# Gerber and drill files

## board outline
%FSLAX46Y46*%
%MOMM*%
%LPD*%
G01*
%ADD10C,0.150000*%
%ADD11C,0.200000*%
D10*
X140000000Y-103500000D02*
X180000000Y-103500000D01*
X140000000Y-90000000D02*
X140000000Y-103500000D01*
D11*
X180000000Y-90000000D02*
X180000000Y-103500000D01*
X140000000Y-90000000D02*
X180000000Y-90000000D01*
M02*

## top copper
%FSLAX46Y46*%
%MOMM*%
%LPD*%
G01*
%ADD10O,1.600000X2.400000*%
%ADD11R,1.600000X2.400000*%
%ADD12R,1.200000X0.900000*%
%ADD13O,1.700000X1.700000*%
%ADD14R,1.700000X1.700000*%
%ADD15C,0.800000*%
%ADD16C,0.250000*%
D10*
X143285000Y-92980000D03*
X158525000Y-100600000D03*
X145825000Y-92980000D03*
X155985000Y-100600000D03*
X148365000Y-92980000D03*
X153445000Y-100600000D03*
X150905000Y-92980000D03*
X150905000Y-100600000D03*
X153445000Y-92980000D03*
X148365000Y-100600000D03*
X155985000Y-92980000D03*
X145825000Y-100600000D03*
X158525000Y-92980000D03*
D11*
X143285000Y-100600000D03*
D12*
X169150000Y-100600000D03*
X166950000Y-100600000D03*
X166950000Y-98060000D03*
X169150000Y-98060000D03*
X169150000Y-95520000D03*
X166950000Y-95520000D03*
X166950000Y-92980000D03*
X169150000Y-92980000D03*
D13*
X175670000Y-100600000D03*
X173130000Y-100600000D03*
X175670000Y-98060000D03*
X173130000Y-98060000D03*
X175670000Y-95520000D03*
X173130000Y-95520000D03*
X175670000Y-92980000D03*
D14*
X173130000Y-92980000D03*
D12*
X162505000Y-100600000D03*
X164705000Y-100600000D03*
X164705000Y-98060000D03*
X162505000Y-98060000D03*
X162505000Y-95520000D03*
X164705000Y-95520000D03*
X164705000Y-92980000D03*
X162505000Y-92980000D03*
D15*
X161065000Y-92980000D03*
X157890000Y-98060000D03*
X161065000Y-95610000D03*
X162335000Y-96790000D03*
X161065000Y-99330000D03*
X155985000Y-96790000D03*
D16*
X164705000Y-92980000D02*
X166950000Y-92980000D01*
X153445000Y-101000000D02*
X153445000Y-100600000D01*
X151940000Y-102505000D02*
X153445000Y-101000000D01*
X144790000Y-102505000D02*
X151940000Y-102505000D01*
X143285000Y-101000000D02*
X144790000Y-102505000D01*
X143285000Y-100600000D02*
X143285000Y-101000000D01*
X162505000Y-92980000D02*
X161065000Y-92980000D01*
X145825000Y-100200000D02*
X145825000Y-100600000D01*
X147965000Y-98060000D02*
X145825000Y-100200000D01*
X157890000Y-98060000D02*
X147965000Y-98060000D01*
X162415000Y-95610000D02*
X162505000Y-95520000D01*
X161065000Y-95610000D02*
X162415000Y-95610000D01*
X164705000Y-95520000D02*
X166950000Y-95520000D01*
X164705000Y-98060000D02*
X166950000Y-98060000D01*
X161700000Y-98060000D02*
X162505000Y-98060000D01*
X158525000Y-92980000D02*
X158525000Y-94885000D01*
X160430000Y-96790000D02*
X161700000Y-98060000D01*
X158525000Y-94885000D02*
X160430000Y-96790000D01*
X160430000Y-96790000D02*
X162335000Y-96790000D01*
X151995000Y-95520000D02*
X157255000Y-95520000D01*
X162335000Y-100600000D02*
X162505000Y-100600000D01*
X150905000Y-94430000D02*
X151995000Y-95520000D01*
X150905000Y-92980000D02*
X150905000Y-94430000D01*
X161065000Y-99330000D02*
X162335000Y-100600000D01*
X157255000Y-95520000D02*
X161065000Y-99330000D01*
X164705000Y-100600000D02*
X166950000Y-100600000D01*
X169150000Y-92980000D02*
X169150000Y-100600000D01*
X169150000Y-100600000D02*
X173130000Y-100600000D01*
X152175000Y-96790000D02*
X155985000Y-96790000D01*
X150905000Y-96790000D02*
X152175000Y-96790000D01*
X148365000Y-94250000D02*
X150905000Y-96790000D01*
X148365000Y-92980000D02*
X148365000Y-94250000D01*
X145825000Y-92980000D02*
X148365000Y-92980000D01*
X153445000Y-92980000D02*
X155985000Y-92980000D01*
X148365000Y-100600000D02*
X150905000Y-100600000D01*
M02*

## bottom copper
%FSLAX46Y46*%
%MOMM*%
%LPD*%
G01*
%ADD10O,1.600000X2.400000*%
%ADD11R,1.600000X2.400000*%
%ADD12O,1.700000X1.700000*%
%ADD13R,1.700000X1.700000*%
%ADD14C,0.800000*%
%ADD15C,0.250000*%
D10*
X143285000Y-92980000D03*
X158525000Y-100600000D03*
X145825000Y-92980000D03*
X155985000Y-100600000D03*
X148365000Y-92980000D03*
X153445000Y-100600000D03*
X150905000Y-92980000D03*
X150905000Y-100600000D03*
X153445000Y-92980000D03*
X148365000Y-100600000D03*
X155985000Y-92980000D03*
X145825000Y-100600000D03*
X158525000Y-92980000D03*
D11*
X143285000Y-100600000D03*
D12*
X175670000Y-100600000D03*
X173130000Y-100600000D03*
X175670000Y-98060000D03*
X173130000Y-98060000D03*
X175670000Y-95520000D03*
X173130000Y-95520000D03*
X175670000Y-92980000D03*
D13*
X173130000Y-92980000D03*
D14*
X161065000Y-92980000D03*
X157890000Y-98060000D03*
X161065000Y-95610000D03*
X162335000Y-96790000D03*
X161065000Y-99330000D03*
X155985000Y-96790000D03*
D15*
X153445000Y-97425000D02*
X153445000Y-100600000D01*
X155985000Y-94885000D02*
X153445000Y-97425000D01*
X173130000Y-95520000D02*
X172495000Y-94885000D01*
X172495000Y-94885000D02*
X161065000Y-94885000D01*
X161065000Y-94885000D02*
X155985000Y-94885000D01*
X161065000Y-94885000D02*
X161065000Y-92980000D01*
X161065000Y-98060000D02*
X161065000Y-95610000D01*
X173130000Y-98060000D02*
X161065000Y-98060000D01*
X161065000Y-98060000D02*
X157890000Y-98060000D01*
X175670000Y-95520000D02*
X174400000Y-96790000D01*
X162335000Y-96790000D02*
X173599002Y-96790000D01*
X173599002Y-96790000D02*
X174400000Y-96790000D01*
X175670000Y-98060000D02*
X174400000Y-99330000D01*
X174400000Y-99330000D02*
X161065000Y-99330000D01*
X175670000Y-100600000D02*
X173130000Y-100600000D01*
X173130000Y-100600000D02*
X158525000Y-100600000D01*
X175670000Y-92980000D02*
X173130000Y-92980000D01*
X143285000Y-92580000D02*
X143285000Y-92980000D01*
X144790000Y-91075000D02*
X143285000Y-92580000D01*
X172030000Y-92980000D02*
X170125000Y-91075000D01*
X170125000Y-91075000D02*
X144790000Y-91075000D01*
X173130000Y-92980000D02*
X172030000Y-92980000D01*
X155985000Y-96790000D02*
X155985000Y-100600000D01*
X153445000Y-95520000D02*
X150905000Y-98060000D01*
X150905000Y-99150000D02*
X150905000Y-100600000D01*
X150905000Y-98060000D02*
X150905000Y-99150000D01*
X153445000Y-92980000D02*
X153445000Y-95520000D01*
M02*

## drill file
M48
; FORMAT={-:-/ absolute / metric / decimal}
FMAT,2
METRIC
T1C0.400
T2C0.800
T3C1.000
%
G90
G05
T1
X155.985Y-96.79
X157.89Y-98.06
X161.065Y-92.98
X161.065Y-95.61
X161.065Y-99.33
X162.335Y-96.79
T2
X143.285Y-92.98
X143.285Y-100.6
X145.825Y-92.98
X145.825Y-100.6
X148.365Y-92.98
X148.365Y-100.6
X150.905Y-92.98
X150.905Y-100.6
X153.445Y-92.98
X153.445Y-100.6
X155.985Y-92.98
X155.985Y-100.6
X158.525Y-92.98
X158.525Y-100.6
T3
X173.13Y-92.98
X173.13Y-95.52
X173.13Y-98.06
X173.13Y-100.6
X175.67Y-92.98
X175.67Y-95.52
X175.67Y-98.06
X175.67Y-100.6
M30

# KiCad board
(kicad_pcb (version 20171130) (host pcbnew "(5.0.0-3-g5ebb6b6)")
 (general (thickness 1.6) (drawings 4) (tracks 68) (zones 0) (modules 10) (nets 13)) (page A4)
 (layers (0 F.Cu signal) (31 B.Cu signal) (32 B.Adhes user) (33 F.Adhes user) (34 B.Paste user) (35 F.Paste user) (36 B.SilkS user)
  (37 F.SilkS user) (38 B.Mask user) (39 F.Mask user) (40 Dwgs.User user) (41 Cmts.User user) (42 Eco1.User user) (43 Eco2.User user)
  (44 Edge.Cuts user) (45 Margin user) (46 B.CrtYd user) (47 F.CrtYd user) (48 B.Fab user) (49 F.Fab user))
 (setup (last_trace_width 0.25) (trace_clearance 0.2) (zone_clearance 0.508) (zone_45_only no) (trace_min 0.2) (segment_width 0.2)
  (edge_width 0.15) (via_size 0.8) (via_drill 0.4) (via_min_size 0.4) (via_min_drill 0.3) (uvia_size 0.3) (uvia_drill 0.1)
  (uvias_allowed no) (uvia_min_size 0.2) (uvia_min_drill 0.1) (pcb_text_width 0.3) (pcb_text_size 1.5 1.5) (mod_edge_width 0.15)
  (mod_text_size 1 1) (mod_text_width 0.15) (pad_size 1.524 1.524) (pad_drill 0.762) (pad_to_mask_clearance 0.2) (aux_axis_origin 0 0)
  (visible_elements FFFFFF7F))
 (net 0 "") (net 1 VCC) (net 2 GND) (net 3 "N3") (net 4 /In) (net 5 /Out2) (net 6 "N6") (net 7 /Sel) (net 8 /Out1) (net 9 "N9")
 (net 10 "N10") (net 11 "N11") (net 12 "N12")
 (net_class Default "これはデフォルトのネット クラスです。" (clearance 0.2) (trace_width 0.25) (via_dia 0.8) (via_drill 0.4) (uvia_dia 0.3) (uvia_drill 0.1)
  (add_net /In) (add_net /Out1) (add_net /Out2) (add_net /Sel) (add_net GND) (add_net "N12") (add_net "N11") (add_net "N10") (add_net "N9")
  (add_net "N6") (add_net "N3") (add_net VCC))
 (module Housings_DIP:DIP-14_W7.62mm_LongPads (layer F.Cu) (at 143.285 100.6 90)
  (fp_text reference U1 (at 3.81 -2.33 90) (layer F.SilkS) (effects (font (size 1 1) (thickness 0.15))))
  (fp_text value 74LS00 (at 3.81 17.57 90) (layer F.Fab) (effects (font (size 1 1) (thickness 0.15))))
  (pad 14 thru_hole oval (at 7.62 0 90) (size 2.4 1.6) (drill 0.8) (layers *.Cu *.Mask) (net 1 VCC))
  (pad 7 thru_hole oval (at 0 15.24 90) (size 2.4 1.6) (drill 0.8) (layers *.Cu *.Mask) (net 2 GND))
  (pad 13 thru_hole oval (at 7.62 2.54 90) (size 2.4 1.6) (drill 0.8) (layers *.Cu *.Mask) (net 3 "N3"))
  (pad 6 thru_hole oval (at 0 12.7 90) (size 2.4 1.6) (drill 0.8) (layers *.Cu *.Mask) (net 3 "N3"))
  (pad 12 thru_hole oval (at 7.62 5.08 90) (size 2.4 1.6) (drill 0.8) (layers *.Cu *.Mask) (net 3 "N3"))
  (pad 5 thru_hole oval (at 0 10.16 90) (size 2.4 1.6) (drill 0.8) (layers *.Cu *.Mask) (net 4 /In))
  (pad 11 thru_hole oval (at 7.62 7.62 90) (size 2.4 1.6) (drill 0.8) (layers *.Cu *.Mask) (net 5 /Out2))
  (pad 4 thru_hole oval (at 0 7.62 90) (size 2.4 1.6) (drill 0.8) (layers *.Cu *.Mask) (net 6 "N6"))
  (pad 10 thru_hole oval (at 7.62 10.16 90) (size 2.4 1.6) (drill 0.8) (layers *.Cu *.Mask) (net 6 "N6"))
  (pad 3 thru_hole oval (at 0 5.08 90) (size 2.4 1.6) (drill 0.8) (layers *.Cu *.Mask) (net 6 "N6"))
  (pad 9 thru_hole oval (at 7.62 12.7 90) (size 2.4 1.6) (drill 0.8) (layers *.Cu *.Mask) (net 6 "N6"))
  (pad 2 thru_hole oval (at 0 2.54 90) (size 2.4 1.6) (drill 0.8) (layers *.Cu *.Mask) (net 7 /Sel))
  (pad 8 thru_hole oval (at 7.62 15.24 90) (size 2.4 1.6) (drill 0.8) (layers *.Cu *.Mask) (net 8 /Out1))
  (pad 1 thru_hole rect (at 0 0 90) (size 2.4 1.6) (drill 0.8) (layers *.Cu *.Mask) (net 4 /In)))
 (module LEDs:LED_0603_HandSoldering (layer F.Cu) (at 168.05 100.6 180)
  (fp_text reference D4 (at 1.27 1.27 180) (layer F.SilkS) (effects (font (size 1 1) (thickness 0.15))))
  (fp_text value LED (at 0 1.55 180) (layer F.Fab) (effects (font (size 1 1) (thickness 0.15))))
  (pad 1 smd rect (at -1.1 0 180) (size 1.2 0.9) (layers F.Cu F.Paste F.Mask) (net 2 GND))
  (pad 2 smd rect (at 1.1 0 180) (size 1.2 0.9) (layers F.Cu F.Paste F.Mask) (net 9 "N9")))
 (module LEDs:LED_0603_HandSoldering (layer F.Cu) (at 168.05 98.06 180)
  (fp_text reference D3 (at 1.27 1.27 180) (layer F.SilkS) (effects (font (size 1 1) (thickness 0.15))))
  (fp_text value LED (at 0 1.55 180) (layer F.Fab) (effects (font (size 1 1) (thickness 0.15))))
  (pad 2 smd rect (at 1.1 0 180) (size 1.2 0.9) (layers F.Cu F.Paste F.Mask) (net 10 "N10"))
  (pad 1 smd rect (at -1.1 0 180) (size 1.2 0.9) (layers F.Cu F.Paste F.Mask) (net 2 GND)))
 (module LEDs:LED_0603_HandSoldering (layer F.Cu) (at 168.05 95.52 180)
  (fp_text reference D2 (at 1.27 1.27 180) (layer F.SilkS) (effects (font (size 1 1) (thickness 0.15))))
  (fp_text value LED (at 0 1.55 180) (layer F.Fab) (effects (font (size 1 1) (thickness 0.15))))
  (pad 1 smd rect (at -1.1 0 180) (size 1.2 0.9) (layers F.Cu F.Paste F.Mask) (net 2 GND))
  (pad 2 smd rect (at 1.1 0 180) (size 1.2 0.9) (layers F.Cu F.Paste F.Mask) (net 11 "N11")))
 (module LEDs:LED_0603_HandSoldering (layer F.Cu) (at 168.05 92.98 180)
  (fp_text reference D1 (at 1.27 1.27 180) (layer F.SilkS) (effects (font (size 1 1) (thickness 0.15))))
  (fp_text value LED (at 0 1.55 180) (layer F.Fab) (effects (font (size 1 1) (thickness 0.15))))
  (pad 2 smd rect (at 1.1 0 180) (size 1.2 0.9) (layers F.Cu F.Paste F.Mask) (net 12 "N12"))
  (pad 1 smd rect (at -1.1 0 180) (size 1.2 0.9) (layers F.Cu F.Paste F.Mask) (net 2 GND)))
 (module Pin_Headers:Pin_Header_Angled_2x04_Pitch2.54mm (layer F.Cu) (at 173.13 92.98)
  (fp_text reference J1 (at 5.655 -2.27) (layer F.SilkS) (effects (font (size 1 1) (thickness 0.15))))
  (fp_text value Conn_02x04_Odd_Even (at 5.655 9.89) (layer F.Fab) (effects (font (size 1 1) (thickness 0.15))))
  (pad 8 thru_hole oval (at 2.54 7.62) (size 1.7 1.7) (drill 1) (layers *.Cu *.Mask) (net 2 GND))
  (pad 7 thru_hole oval (at 0 7.62) (size 1.7 1.7) (drill 1) (layers *.Cu *.Mask) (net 2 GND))
  (pad 6 thru_hole oval (at 2.54 5.08) (size 1.7 1.7) (drill 1) (layers *.Cu *.Mask) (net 5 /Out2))
  (pad 5 thru_hole oval (at 0 5.08) (size 1.7 1.7) (drill 1) (layers *.Cu *.Mask) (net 7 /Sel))
  (pad 4 thru_hole oval (at 2.54 2.54) (size 1.7 1.7) (drill 1) (layers *.Cu *.Mask) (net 8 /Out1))
  (pad 3 thru_hole oval (at 0 2.54) (size 1.7 1.7) (drill 1) (layers *.Cu *.Mask) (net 4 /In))
  (pad 2 thru_hole oval (at 2.54 0) (size 1.7 1.7) (drill 1) (layers *.Cu *.Mask) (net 1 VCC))
  (pad 1 thru_hole rect (at 0 0) (size 1.7 1.7) (drill 1) (layers *.Cu *.Mask) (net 1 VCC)))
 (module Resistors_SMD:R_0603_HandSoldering (layer F.Cu) (at 163.605 100.6)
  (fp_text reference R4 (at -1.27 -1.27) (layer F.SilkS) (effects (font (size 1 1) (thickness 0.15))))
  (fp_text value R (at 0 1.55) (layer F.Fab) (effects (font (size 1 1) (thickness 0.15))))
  (pad 1 smd rect (at -1.1 0) (size 1.2 0.9) (layers F.Cu F.Paste F.Mask) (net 5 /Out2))
  (pad 2 smd rect (at 1.1 0) (size 1.2 0.9) (layers F.Cu F.Paste F.Mask) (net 9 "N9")))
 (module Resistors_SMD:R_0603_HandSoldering (layer F.Cu) (at 163.605 98.06)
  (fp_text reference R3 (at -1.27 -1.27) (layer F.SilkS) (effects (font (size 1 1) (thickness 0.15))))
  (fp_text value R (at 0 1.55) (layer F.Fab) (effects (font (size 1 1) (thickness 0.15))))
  (pad 2 smd rect (at 1.1 0) (size 1.2 0.9) (layers F.Cu F.Paste F.Mask) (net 10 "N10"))
  (pad 1 smd rect (at -1.1 0) (size 1.2 0.9) (layers F.Cu F.Paste F.Mask) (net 8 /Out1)))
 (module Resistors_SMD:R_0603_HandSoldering (layer F.Cu) (at 163.605 95.52)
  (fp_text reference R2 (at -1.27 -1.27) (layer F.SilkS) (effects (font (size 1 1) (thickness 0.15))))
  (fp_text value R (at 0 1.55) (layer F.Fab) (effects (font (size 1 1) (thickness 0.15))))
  (pad 1 smd rect (at -1.1 0) (size 1.2 0.9) (layers F.Cu F.Paste F.Mask) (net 7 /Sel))
  (pad 2 smd rect (at 1.1 0) (size 1.2 0.9) (layers F.Cu F.Paste F.Mask) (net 11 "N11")))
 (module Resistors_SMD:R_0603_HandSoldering (layer F.Cu) (at 163.605 92.98)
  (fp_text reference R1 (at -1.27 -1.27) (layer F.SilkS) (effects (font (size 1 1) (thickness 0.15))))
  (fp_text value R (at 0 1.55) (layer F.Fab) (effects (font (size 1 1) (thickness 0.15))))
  (pad 2 smd rect (at 1.1 0) (size 1.2 0.9) (layers F.Cu F.Paste F.Mask) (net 12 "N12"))
  (pad 1 smd rect (at -1.1 0) (size 1.2 0.9) (layers F.Cu F.Paste F.Mask) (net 4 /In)))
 (gr_line (start 140 103.5) (end 180 103.5) (layer Edge.Cuts) (width 0.15))
 (gr_line (start 140 90) (end 140 103.5) (layer Edge.Cuts) (width 0.15))
 (gr_line (start 180 90) (end 180 103.5) (layer Edge.Cuts) (width 0.2))
 (gr_line (start 140 90) (end 180 90) (layer Edge.Cuts) (width 0.2))
 (segment (start 164.705 92.98) (end 166.95 92.98) (width 0.25) (layer F.Cu) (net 12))
 (segment (start 153.445 101) (end 153.445 100.6) (width 0.25) (layer F.Cu) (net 4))
 (segment (start 151.94 102.505) (end 153.445 101) (width 0.25) (layer F.Cu) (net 4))
 (segment (start 144.79 102.505) (end 151.94 102.505) (width 0.25) (layer F.Cu) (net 4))
 (segment (start 143.285 101) (end 144.79 102.505) (width 0.25) (layer F.Cu) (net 4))
 (segment (start 143.285 100.6) (end 143.285 101) (width 0.25) (layer F.Cu) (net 4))
 (segment (start 153.445 97.425) (end 153.445 100.6) (width 0.25) (layer B.Cu) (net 4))
 (segment (start 155.985 94.885) (end 153.445 97.425) (width 0.25) (layer B.Cu) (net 4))
 (segment (start 173.13 95.52) (end 172.495 94.885) (width 0.25) (layer B.Cu) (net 4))
 (segment (start 172.495 94.885) (end 161.065 94.885) (width 0.25) (layer B.Cu) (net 4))
 (segment (start 161.065 94.885) (end 155.985 94.885) (width 0.25) (layer B.Cu) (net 4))
 (via (at 161.065 92.98) (size 0.8) (drill 0.4) (layers F.Cu B.Cu) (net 4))
 (segment (start 161.065 94.885) (end 161.065 92.98) (width 0.25) (layer B.Cu) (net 4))
 (segment (start 162.505 92.98) (end 161.065 92.98) (width 0.25) (layer F.Cu) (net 4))
 (via (at 157.89 98.06) (size 0.8) (drill 0.4) (layers F.Cu B.Cu) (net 7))
 (segment (start 145.825 100.2) (end 145.825 100.6) (width 0.25) (layer F.Cu) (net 7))
 (segment (start 147.965 98.06) (end 145.825 100.2) (width 0.25) (layer F.Cu) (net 7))
 (segment (start 157.89 98.06) (end 147.965 98.06) (width 0.25) (layer F.Cu) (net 7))
 (via (at 161.065 95.61) (size 0.8) (drill 0.4) (layers F.Cu B.Cu) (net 7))
 (segment (start 161.065 98.06) (end 161.065 95.61) (width 0.25) (layer B.Cu) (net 7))
 (segment (start 173.13 98.06) (end 161.065 98.06) (width 0.25) (layer B.Cu) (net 7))
 (segment (start 161.065 98.06) (end 157.89 98.06) (width 0.25) (layer B.Cu) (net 7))
 (segment (start 162.415 95.61) (end 162.505 95.52) (width 0.25) (layer F.Cu) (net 7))
 (segment (start 161.065 95.61) (end 162.415 95.61) (width 0.25) (layer F.Cu) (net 7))
 (segment (start 164.705 95.52) (end 166.95 95.52) (width 0.25) (layer F.Cu) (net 11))
 (segment (start 164.705 98.06) (end 166.95 98.06) (width 0.25) (layer F.Cu) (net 10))
 (segment (start 161.7 98.06) (end 162.505 98.06) (width 0.25) (layer F.Cu) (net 8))
 (segment (start 158.525 92.98) (end 158.525 94.885) (width 0.25) (layer F.Cu) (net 8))
 (segment (start 175.67 95.52) (end 174.4 96.79) (width 0.25) (layer B.Cu) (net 8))
 (segment (start 160.43 96.79) (end 161.7 98.06) (width 0.25) (layer F.Cu) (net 8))
 (segment (start 158.525 94.885) (end 160.43 96.79) (width 0.25) (layer F.Cu) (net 8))
 (via (at 162.335 96.79) (size 0.8) (drill 0.4) (layers F.Cu B.Cu) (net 8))
 (segment (start 160.43 96.79) (end 162.335 96.79) (width 0.25) (layer F.Cu) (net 8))
 (segment (start 162.335 96.79) (end 173.599002 96.79) (width 0.25) (layer B.Cu) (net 8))
 (segment (start 173.599002 96.79) (end 174.4 96.79) (width 0.25) (layer B.Cu) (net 8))
 (segment (start 151.995 95.52) (end 157.255 95.52) (width 0.25) (layer F.Cu) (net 5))
 (segment (start 162.335 100.6) (end 162.505 100.6) (width 0.25) (layer F.Cu) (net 5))
 (segment (start 150.905 94.43) (end 151.995 95.52) (width 0.25) (layer F.Cu) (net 5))
 (segment (start 150.905 92.98) (end 150.905 94.43) (width 0.25) (layer F.Cu) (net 5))
 (segment (start 175.67 98.06) (end 174.4 99.33) (width 0.25) (layer B.Cu) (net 5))
 (via (at 161.065 99.33) (size 0.8) (drill 0.4) (layers F.Cu B.Cu) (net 5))
 (segment (start 161.065 99.33) (end 162.335 100.6) (width 0.25) (layer F.Cu) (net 5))
 (segment (start 174.4 99.33) (end 161.065 99.33) (width 0.25) (layer B.Cu) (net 5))
 (segment (start 157.255 95.52) (end 161.065 99.33) (width 0.25) (layer F.Cu) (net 5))
 (segment (start 164.705 100.6) (end 166.95 100.6) (width 0.25) (layer F.Cu) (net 9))
 (segment (start 175.67 100.6) (end 173.13 100.6) (width 0.25) (layer B.Cu) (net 2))
 (segment (start 169.15 92.98) (end 169.15 100.6) (width 0.25) (layer F.Cu) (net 2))
 (segment (start 169.15 100.6) (end 173.13 100.6) (width 0.25) (layer F.Cu) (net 2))
 (segment (start 173.13 100.6) (end 158.525 100.6) (width 0.25) (layer B.Cu) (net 2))
 (segment (start 175.67 92.98) (end 173.13 92.98) (width 0.25) (layer B.Cu) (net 1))
 (segment (start 143.285 92.58) (end 143.285 92.98) (width 0.25) (layer B.Cu) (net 1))
 (segment (start 144.79 91.075) (end 143.285 92.58) (width 0.25) (layer B.Cu) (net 1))
 (segment (start 172.03 92.98) (end 170.125 91.075) (width 0.25) (layer B.Cu) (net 1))
 (segment (start 170.125 91.075) (end 144.79 91.075) (width 0.25) (layer B.Cu) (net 1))
 (segment (start 173.13 92.98) (end 172.03 92.98) (width 0.25) (layer B.Cu) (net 1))
 (via (at 155.985 96.79) (size 0.8) (drill 0.4) (layers F.Cu B.Cu) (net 3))
 (segment (start 155.985 96.79) (end 155.985 100.6) (width 0.25) (layer B.Cu) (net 3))
 (segment (start 152.175 96.79) (end 155.985 96.79) (width 0.25) (layer F.Cu) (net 3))
 (segment (start 150.905 96.79) (end 152.175 96.79) (width 0.25) (layer F.Cu) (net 3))
 (segment (start 148.365 94.25) (end 150.905 96.79) (width 0.25) (layer F.Cu) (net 3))
 (segment (start 148.365 92.98) (end 148.365 94.25) (width 0.25) (layer F.Cu) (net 3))
 (segment (start 145.825 92.98) (end 148.365 92.98) (width 0.25) (layer F.Cu) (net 3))
 (segment (start 153.445 92.98) (end 155.985 92.98) (width 0.25) (layer F.Cu) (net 6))
 (segment (start 148.365 100.6) (end 150.905 100.6) (width 0.25) (layer F.Cu) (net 6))
 (segment (start 153.445 95.52) (end 150.905 98.06) (width 0.25) (layer B.Cu) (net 6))
 (segment (start 150.905 99.15) (end 150.905 100.6) (width 0.25) (layer B.Cu) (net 6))
 (segment (start 150.905 98.06) (end 150.905 99.15) (width 0.25) (layer B.Cu) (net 6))
 (segment (start 153.445 92.98) (end 153.445 95.52) (width 0.25) (layer B.Cu) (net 6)))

